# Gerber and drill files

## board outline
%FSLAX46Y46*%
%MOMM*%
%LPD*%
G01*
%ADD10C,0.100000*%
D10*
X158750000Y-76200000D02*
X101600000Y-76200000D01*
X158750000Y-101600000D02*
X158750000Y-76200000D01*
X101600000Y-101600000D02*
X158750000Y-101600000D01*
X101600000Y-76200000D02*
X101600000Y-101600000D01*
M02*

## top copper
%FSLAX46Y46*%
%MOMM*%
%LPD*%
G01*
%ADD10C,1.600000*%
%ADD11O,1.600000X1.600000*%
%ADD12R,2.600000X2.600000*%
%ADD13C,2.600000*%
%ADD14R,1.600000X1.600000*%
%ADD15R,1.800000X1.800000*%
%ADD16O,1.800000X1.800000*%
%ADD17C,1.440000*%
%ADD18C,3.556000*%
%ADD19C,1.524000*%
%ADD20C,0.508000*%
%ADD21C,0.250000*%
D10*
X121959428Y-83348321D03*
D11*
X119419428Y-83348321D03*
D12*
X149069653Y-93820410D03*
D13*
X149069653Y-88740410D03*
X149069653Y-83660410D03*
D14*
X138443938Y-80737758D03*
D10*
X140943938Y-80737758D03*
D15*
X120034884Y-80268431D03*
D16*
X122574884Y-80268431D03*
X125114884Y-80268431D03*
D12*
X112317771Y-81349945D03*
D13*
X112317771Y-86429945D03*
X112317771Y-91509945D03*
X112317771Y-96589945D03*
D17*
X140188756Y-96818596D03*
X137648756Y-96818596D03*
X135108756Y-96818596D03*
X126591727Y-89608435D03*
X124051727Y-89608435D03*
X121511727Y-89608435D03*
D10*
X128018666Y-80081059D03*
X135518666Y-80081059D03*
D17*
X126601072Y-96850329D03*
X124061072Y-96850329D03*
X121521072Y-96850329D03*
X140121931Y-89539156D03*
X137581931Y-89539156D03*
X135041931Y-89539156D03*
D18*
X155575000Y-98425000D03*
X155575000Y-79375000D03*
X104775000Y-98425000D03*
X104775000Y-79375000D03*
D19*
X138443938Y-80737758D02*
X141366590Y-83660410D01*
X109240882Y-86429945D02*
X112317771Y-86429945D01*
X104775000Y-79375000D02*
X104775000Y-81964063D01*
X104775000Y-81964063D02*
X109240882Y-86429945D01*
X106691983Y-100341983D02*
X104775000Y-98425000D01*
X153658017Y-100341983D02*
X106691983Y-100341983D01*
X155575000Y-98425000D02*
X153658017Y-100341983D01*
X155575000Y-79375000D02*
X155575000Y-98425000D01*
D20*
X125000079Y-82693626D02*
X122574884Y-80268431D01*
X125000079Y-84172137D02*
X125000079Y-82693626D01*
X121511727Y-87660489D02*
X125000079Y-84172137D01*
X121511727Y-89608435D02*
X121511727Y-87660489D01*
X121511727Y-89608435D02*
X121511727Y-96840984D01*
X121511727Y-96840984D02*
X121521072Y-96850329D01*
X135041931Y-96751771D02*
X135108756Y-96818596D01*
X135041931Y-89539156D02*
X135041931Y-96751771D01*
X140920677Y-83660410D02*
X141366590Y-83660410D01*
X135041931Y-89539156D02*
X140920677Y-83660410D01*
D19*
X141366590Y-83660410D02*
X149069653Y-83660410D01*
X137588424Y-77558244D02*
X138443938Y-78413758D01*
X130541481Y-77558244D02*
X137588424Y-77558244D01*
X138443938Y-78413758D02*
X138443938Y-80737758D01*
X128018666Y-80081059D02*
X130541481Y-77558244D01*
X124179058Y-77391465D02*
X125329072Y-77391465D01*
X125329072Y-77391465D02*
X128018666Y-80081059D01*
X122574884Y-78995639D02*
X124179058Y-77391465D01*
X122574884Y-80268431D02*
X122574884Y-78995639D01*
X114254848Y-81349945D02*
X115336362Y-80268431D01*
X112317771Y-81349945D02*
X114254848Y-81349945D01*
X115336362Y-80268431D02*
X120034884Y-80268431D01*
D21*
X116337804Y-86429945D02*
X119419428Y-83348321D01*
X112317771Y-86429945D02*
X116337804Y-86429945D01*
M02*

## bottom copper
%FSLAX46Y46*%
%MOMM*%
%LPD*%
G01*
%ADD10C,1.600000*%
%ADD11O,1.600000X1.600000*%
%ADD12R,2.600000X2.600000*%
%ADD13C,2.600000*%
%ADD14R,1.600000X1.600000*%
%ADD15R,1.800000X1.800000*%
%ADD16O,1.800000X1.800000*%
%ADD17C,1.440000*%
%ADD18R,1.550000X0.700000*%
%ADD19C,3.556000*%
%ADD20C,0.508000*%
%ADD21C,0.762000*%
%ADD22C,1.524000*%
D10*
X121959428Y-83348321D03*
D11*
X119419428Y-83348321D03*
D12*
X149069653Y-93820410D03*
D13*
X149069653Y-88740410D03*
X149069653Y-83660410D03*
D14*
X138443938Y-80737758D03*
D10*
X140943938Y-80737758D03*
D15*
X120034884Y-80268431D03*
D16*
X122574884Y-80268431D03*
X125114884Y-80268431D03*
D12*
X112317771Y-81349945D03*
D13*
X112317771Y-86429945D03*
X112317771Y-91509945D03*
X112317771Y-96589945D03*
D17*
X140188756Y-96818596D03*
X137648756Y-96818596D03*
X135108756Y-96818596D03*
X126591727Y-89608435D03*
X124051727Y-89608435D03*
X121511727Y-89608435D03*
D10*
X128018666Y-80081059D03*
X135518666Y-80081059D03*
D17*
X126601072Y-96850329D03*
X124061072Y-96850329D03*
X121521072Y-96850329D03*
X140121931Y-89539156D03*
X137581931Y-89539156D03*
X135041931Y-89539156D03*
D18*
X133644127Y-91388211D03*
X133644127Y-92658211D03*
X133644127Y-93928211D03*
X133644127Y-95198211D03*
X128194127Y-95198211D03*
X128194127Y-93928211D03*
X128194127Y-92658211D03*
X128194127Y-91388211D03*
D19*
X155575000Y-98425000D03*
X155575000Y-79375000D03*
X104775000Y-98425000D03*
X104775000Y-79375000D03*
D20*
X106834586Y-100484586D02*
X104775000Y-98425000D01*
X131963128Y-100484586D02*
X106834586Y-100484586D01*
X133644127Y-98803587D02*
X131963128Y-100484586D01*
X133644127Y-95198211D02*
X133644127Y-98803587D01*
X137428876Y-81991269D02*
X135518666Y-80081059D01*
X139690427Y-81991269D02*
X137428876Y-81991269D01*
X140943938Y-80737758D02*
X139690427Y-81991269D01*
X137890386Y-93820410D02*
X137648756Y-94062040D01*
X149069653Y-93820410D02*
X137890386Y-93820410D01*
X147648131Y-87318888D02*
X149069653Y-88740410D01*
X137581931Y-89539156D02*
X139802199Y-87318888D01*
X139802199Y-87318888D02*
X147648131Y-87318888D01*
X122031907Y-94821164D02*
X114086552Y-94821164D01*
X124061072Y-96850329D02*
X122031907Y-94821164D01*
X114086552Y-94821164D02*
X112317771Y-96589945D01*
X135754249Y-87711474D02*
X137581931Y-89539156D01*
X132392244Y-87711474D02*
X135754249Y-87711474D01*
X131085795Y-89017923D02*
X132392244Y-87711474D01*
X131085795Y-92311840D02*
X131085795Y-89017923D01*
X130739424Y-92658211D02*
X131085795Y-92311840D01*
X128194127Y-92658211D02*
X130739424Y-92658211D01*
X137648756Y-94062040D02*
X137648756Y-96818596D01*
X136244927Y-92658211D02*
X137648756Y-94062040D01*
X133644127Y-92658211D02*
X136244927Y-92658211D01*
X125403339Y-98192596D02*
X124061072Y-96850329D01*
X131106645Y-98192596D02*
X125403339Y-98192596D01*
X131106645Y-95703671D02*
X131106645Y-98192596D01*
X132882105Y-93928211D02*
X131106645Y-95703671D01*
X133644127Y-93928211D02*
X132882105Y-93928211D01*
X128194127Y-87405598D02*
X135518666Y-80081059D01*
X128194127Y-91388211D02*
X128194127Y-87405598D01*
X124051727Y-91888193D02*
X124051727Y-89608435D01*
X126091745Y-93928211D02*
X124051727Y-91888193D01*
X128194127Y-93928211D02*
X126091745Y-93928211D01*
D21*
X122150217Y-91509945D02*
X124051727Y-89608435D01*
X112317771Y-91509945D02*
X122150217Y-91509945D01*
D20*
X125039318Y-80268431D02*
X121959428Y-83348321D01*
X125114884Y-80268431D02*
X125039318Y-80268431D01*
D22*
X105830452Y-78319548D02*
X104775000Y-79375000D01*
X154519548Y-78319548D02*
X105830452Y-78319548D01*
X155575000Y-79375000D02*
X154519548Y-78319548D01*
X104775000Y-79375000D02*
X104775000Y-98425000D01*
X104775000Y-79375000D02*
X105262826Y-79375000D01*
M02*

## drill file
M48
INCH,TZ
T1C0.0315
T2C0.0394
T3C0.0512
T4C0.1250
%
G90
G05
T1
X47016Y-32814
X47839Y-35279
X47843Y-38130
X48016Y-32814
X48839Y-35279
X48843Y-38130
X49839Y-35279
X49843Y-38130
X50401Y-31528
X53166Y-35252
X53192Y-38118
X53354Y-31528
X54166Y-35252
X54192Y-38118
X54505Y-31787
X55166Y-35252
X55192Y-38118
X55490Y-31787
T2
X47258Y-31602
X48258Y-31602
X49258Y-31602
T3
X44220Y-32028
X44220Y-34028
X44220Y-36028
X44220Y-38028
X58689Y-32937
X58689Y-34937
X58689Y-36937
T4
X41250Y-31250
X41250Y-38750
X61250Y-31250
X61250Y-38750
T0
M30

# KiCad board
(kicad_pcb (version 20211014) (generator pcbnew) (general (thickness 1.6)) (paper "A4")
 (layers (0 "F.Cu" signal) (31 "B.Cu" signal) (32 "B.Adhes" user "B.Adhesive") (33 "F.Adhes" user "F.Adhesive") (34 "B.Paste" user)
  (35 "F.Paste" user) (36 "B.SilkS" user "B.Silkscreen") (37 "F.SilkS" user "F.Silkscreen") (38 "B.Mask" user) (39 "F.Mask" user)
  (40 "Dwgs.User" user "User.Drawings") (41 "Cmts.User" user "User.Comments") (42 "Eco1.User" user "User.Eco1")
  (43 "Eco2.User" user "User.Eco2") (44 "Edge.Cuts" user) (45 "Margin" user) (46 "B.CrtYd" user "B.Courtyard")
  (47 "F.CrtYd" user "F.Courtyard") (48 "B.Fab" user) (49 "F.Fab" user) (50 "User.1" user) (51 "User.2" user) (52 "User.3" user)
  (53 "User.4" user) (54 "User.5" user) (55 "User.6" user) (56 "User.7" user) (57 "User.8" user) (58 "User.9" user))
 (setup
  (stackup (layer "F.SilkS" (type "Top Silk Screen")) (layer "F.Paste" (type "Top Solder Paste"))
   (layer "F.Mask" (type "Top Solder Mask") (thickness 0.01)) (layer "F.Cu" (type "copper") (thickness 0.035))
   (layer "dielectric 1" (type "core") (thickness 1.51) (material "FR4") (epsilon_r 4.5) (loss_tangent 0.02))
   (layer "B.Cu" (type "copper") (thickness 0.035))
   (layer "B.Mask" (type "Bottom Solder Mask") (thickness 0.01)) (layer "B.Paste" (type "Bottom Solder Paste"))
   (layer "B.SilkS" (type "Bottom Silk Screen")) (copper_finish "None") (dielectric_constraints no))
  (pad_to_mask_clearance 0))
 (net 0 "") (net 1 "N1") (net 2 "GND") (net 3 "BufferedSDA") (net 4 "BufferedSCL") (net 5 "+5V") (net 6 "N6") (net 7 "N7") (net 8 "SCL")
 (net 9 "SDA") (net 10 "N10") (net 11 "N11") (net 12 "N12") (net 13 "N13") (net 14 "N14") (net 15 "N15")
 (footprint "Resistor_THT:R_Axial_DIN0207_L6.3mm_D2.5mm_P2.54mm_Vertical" (layer "F.Cu") (at 121.959428 83.348321 180)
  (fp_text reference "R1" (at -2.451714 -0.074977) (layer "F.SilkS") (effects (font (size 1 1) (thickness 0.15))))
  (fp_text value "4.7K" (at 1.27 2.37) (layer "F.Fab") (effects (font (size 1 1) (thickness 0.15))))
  (pad "1" thru_hole circle locked (at 0 0 180) (size 1.6 1.6) (drill 0.8) (layers *.Cu *.Mask) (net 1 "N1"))
  (pad "2" thru_hole oval locked (at 2.54 0 180) (size 1.6 1.6) (drill 0.8) (layers *.Cu *.Mask) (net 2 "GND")))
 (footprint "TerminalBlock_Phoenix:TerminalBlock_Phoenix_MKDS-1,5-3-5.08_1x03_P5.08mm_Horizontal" (layer "F.Cu") (at 149.069653 93.82041 90)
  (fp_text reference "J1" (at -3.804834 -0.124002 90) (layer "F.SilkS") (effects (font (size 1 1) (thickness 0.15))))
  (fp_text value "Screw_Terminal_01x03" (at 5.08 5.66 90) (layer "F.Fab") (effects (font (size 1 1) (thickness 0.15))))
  (pad "1" thru_hole rect locked (at 0 0 90) (size 2.6 2.6) (drill 1.3) (layers *.Cu *.Mask) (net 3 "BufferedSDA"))
  (pad "2" thru_hole circle locked (at 5.08 0 90) (size 2.6 2.6) (drill 1.3) (layers *.Cu *.Mask) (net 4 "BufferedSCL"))
  (pad "3" thru_hole circle locked (at 10.16 0 90) (size 2.6 2.6) (drill 1.3) (layers *.Cu *.Mask) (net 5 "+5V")))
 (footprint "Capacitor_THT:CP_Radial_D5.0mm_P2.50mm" (layer "F.Cu") (at 138.443938 80.737758)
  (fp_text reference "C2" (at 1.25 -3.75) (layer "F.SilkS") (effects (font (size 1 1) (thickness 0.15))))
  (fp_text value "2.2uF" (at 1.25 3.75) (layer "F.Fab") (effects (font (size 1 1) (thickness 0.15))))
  (pad "1" thru_hole rect locked (at 0 0) (size 1.6 1.6) (drill 0.8) (layers *.Cu *.Mask) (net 5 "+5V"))
  (pad "2" thru_hole circle locked (at 2.5 0) (size 1.6 1.6) (drill 0.8) (layers *.Cu *.Mask) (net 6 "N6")))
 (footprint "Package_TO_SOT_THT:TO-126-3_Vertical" (layer "F.Cu") (at 120.034884 80.268431)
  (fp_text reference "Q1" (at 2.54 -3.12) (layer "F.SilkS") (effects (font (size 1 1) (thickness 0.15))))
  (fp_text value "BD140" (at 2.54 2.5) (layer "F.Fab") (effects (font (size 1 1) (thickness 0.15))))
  (pad "1" thru_hole rect locked (at 0 0) (size 1.8 1.8) (drill 1) (layers *.Cu *.Mask) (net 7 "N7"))
  (pad "2" thru_hole oval locked (at 2.54 0) (size 1.8 1.8) (drill 1) (layers *.Cu *.Mask) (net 5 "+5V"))
  (pad "3" thru_hole oval locked (at 5.08 0) (size 1.8 1.8) (drill 1) (layers *.Cu *.Mask) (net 1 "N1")))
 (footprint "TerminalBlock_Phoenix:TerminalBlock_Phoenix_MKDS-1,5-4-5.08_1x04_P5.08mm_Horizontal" (layer "F.Cu")
  (at 112.317771 81.349945 -90)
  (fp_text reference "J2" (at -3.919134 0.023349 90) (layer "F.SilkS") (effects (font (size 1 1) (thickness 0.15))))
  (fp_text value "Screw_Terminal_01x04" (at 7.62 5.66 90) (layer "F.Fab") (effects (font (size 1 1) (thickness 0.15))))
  (pad "1" thru_hole rect locked (at 0 0 270) (size 2.6 2.6) (drill 1.3) (layers *.Cu *.Mask) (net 7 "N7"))
  (pad "2" thru_hole circle locked (at 5.08 0 270) (size 2.6 2.6) (drill 1.3) (layers *.Cu *.Mask) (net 2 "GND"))
  (pad "3" thru_hole circle locked (at 10.16 0 270) (size 2.6 2.6) (drill 1.3) (layers *.Cu *.Mask) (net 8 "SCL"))
  (pad "4" thru_hole circle locked (at 15.24 0 270) (size 2.6 2.6) (drill 1.3) (layers *.Cu *.Mask) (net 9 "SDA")))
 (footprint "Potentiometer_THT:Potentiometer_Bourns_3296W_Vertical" (layer "F.Cu") (at 140.188756 96.818596)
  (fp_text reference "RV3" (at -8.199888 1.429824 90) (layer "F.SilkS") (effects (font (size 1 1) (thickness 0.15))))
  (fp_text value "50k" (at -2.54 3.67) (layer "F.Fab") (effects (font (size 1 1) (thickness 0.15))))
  (pad "1" thru_hole circle locked (at 0 0) (size 1.44 1.44) (drill 0.8) (layers *.Cu *.Mask) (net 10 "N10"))
  (pad "2" thru_hole circle locked (at -2.54 0) (size 1.44 1.44) (drill 0.8) (layers *.Cu *.Mask) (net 3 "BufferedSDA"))
  (pad "3" thru_hole circle locked (at -5.08 0) (size 1.44 1.44) (drill 0.8) (layers *.Cu *.Mask) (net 5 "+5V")))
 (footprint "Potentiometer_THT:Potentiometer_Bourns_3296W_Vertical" (layer "F.Cu") (at 126.591727 89.608435)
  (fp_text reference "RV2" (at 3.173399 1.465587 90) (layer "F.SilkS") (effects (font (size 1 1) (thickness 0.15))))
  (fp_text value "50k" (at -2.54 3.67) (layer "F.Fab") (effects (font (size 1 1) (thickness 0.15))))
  (pad "1" thru_hole circle locked (at 0 0) (size 1.44 1.44) (drill 0.8) (layers *.Cu *.Mask) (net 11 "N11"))
  (pad "2" thru_hole circle locked (at -2.54 0) (size 1.44 1.44) (drill 0.8) (layers *.Cu *.Mask) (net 8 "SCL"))
  (pad "3" thru_hole circle locked (at -5.08 0) (size 1.44 1.44) (drill 0.8) (layers *.Cu *.Mask) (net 5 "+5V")))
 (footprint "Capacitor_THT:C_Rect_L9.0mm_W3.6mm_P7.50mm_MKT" (layer "F.Cu") (at 128.018666 80.081059)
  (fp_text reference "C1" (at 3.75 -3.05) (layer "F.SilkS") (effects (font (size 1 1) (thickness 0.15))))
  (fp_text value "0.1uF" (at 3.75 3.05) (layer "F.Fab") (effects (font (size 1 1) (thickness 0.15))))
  (pad "1" thru_hole circle locked (at 0 0) (size 1.6 1.6) (drill 0.8) (layers *.Cu *.Mask) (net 5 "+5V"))
  (pad "2" thru_hole circle locked (at 7.5 0) (size 1.6 1.6) (drill 0.8) (layers *.Cu *.Mask) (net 6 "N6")))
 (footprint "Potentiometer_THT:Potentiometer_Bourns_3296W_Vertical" (layer "F.Cu") (at 126.601072 96.850329)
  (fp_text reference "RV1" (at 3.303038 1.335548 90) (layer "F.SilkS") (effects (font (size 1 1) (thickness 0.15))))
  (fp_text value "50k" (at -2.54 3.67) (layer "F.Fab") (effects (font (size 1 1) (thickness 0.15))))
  (pad "1" thru_hole circle locked (at 0 0) (size 1.44 1.44) (drill 0.8) (layers *.Cu *.Mask) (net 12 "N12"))
  (pad "2" thru_hole circle locked (at -2.54 0) (size 1.44 1.44) (drill 0.8) (layers *.Cu *.Mask) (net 9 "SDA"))
  (pad "3" thru_hole circle locked (at -5.08 0) (size 1.44 1.44) (drill 0.8) (layers *.Cu *.Mask) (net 5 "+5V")))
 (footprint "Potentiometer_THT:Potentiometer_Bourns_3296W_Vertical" (layer "F.Cu") (at 140.121931 89.539156)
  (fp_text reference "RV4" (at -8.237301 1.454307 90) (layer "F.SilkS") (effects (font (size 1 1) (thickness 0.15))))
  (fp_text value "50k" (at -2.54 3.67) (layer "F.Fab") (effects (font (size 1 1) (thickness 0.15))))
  (pad "1" thru_hole circle locked (at 0 0) (size 1.44 1.44) (drill 0.8) (layers *.Cu *.Mask) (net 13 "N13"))
  (pad "2" thru_hole circle locked (at -2.54 0) (size 1.44 1.44) (drill 0.8) (layers *.Cu *.Mask) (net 4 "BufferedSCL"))
  (pad "3" thru_hole circle locked (at -5.08 0) (size 1.44 1.44) (drill 0.8) (layers *.Cu *.Mask) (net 5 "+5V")))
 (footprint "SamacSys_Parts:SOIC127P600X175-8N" (layer "B.Cu") (at 130.919127 93.293211 180)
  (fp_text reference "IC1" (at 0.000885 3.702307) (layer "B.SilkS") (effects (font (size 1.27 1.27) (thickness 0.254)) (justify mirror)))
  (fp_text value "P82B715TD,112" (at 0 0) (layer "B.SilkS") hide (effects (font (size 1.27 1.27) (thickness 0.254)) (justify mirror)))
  (pad "1" smd rect locked (at -2.725 1.905 90) (size 0.7 1.55) (layers "B.Cu" "B.Paste" "B.Mask") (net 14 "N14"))
  (pad "2" smd rect locked (at -2.725 0.635 90) (size 0.7 1.55) (layers "B.Cu" "B.Paste" "B.Mask") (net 3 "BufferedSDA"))
  (pad "3" smd rect locked (at -2.725 -0.635 90) (size 0.7 1.55) (layers "B.Cu" "B.Paste" "B.Mask") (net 9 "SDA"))
  (pad "4" smd rect locked (at -2.725 -1.905 90) (size 0.7 1.55) (layers "B.Cu" "B.Paste" "B.Mask") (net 2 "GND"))
  (pad "5" smd rect locked (at 2.725 -1.905 90) (size 0.7 1.55) (layers "B.Cu" "B.Paste" "B.Mask") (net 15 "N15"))
  (pad "6" smd rect locked (at 2.725 -0.635 90) (size 0.7 1.55) (layers "B.Cu" "B.Paste" "B.Mask") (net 8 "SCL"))
  (pad "7" smd rect locked (at 2.725 0.635 90) (size 0.7 1.55) (layers "B.Cu" "B.Paste" "B.Mask") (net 4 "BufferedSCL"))
  (pad "8" smd rect locked (at 2.725 1.905 90) (size 0.7 1.55) (layers "B.Cu" "B.Paste" "B.Mask") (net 6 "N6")))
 (gr_line (start 101.6 76.2) (end 101.6 101.6) (layer "Edge.Cuts") (width 0.1))
 (gr_line (start 158.75 76.2) (end 101.6 76.2) (layer "Edge.Cuts") (width 0.1))
 (gr_line (start 101.6 101.6) (end 158.75 101.6) (layer "Edge.Cuts") (width 0.1))
 (gr_line (start 158.75 101.6) (end 158.75 76.2) (layer "Edge.Cuts") (width 0.1))
 (segment (start 140.920677 83.66041) (end 141.36659 83.66041) (width 0.508) (layer "F.Cu") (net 5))
 (segment (start 128.018666 80.081059) (end 130.541481 77.558244) (width 1.524) (layer "F.Cu") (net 5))
 (segment (start 122.574884 78.995639) (end 124.179058 77.391465) (width 1.524) (layer "F.Cu") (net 5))
 (segment (start 135.041931 96.751771) (end 135.108756 96.818596) (width 0.508) (layer "F.Cu") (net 5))
 (segment (start 125.000079 84.172137) (end 125.000079 82.693626) (width 0.508) (layer "F.Cu") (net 5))
 (segment (start 125.329072 77.391465) (end 128.018666 80.081059) (width 1.524) (layer "F.Cu") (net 5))
 (segment (start 138.443938 78.413758) (end 138.443938 80.737758) (width 1.524) (layer "F.Cu") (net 5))
 (segment (start 130.541481 77.558244) (end 137.588424 77.558244) (width 1.524) (layer "F.Cu") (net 5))
 (segment (start 124.179058 77.391465) (end 125.329072 77.391465) (width 1.524) (layer "F.Cu") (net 5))
 (segment (start 121.511727 96.840984) (end 121.521072 96.850329) (width 0.508) (layer "F.Cu") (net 5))
 (segment (start 121.511727 87.660489) (end 125.000079 84.172137) (width 0.508) (layer "F.Cu") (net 5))
 (segment (start 125.000079 82.693626) (end 122.574884 80.268431) (width 0.508) (layer "F.Cu") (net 5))
 (segment (start 137.588424 77.558244) (end 138.443938 78.413758) (width 1.524) (layer "F.Cu") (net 5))
 (segment (start 135.041931 89.539156) (end 140.920677 83.66041) (width 0.508) (layer "F.Cu") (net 5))
 (segment (start 141.36659 83.66041) (end 149.069653 83.66041) (width 1.524) (layer "F.Cu") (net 5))
 (segment (start 121.511727 89.608435) (end 121.511727 87.660489) (width 0.508) (layer "F.Cu") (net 5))
 (segment (start 135.041931 89.539156) (end 135.041931 96.751771) (width 0.508) (layer "F.Cu") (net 5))
 (segment (start 121.511727 89.608435) (end 121.511727 96.840984) (width 0.508) (layer "F.Cu") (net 5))
 (segment (start 138.443938 80.737758) (end 141.36659 83.66041) (width 1.524) (layer "F.Cu") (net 5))
 (segment (start 122.574884 80.268431) (end 122.574884 78.995639) (width 1.524) (layer "F.Cu") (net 5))
 (segment (start 140.943938 80.737758) (end 139.690427 81.991269) (width 0.508) (layer "B.Cu") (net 6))
 (segment (start 137.428876 81.991269) (end 135.518666 80.081059) (width 0.508) (layer "B.Cu") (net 6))
 (segment (start 128.194127 91.388211) (end 128.194127 87.405598) (width 0.508) (layer "B.Cu") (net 6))
 (segment (start 139.690427 81.991269) (end 137.428876 81.991269) (width 0.508) (layer "B.Cu") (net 6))
 (segment (start 128.194127 87.405598) (end 135.518666 80.081059) (width 0.508) (layer "B.Cu") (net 6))
 (segment (start 149.069653 93.82041) (end 137.890386 93.82041) (width 0.508) (layer "B.Cu") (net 3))
 (segment (start 137.890386 93.82041) (end 137.648756 94.06204) (width 0.508) (layer "B.Cu") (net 3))
 (segment (start 137.648756 94.06204) (end 137.648756 96.818596) (width 0.508) (layer "B.Cu") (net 3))
 (segment (start 136.244927 92.658211) (end 137.648756 94.06204) (width 0.508) (layer "B.Cu") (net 3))
 (segment (start 133.644127 92.658211) (end 136.244927 92.658211) (width 0.508) (layer "B.Cu") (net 3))
 (segment (start 132.882105 93.928211) (end 131.106645 95.703671) (width 0.508) (layer "B.Cu") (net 9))
 (segment (start 124.061072 96.850329) (end 122.031907 94.821164) (width 0.508) (layer "B.Cu") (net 9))
 (segment (start 122.031907 94.821164) (end 114.086552 94.821164) (width 0.508) (layer "B.Cu") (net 9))
 (segment (start 125.403339 98.192596) (end 124.061072 96.850329) (width 0.508) (layer "B.Cu") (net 9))
 (segment (start 114.086552 94.821164) (end 112.317771 96.589945) (width 0.508) (layer "B.Cu") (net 9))
 (segment (start 133.644127 93.928211) (end 132.882105 93.928211) (width 0.508) (layer "B.Cu") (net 9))
 (segment (start 131.106645 95.703671) (end 131.106645 98.192596) (width 0.508) (layer "B.Cu") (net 9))
 (segment (start 131.106645 98.192596) (end 125.403339 98.192596) (width 0.508) (layer "B.Cu") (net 9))
 (segment (start 104.775 81.964063) (end 109.240882 86.429945) (width 1.524) (layer "F.Cu") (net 2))
 (segment (start 112.317771 86.429945) (end 116.337804 86.429945) (width 0.25) (layer "F.Cu") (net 2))
 (segment (start 153.658017 100.341983) (end 106.691983 100.341983) (width 1.524) (layer "F.Cu") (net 2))
 (segment (start 155.575 79.375) (end 155.575 98.425) (width 1.524) (layer "F.Cu") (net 2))
 (segment (start 104.775 79.375) (end 104.775 81.964063) (width 1.524) (layer "F.Cu") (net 2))
 (segment (start 106.691983 100.341983) (end 104.775 98.425) (width 1.524) (layer "F.Cu") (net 2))
 (segment (start 109.240882 86.429945) (end 112.317771 86.429945) (width 1.524) (layer "F.Cu") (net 2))
 (segment (start 116.337804 86.429945) (end 119.419428 83.348321) (width 0.25) (layer "F.Cu") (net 2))
 (segment (start 155.575 98.425) (end 153.658017 100.341983) (width 1.524) (layer "F.Cu") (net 2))
 (via (at 155.575 98.425) (size 3.556) (drill 3.175) (layers "F.Cu" "B.Cu") (free) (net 2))
 (via (at 104.775 79.375) (size 3.556) (drill 3.175) (layers "F.Cu" "B.Cu") (free) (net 2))
 (via (at 104.775 98.425) (size 3.556) (drill 3.175) (layers "F.Cu" "B.Cu") (free) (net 2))
 (via (at 155.575 79.375) (size 3.556) (drill 3.175) (layers "F.Cu" "B.Cu") (free) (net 2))
 (segment (start 104.775 79.375) (end 105.262826 79.375) (width 1.524) (layer "B.Cu") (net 2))
 (segment (start 133.644127 98.803587) (end 131.963128 100.484586) (width 0.508) (layer "B.Cu") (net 2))
 (segment (start 131.963128 100.484586) (end 106.834586 100.484586) (width 0.508) (layer "B.Cu") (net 2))
 (segment (start 155.575 79.375) (end 154.519548 78.319548) (width 1.524) (layer "B.Cu") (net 2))
 (segment (start 106.834586 100.484586) (end 104.775 98.425) (width 0.508) (layer "B.Cu") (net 2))
 (segment (start 133.644127 95.198211) (end 133.644127 98.803587) (width 0.508) (layer "B.Cu") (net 2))
 (segment (start 104.775 79.375) (end 104.775 98.425) (width 1.524) (layer "B.Cu") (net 2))
 (segment (start 105.830452 78.319548) (end 104.775 79.375) (width 1.524) (layer "B.Cu") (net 2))
 (segment (start 154.519548 78.319548) (end 105.830452 78.319548) (width 1.524) (layer "B.Cu") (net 2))
 (segment (start 112.317771 91.509945) (end 122.150217 91.509945) (width 0.762) (layer "B.Cu") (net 8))
 (segment (start 122.150217 91.509945) (end 124.051727 89.608435) (width 0.762) (layer "B.Cu") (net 8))
 (segment (start 124.051727 91.888193) (end 124.051727 89.608435) (width 0.508) (layer "B.Cu") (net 8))
 (segment (start 126.091745 93.928211) (end 124.051727 91.888193) (width 0.508) (layer "B.Cu") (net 8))
 (segment (start 128.194127 93.928211) (end 126.091745 93.928211) (width 0.508) (layer "B.Cu") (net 8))
 (segment (start 130.739424 92.658211) (end 131.085795 92.31184) (width 0.508) (layer "B.Cu") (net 4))
 (segment (start 128.194127 92.658211) (end 130.739424 92.658211) (width 0.508) (layer "B.Cu") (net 4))
 (segment (start 131.085795 89.017923) (end 132.392244 87.711474) (width 0.508) (layer "B.Cu") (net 4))
 (segment (start 147.648131 87.318888) (end 149.069653 88.74041) (width 0.508) (layer "B.Cu") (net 4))
 (segment (start 135.754249 87.711474) (end 137.581931 89.539156) (width 0.508) (layer "B.Cu") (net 4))
 (segment (start 137.581931 89.539156) (end 139.802199 87.318888) (width 0.508) (layer "B.Cu") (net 4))
 (segment (start 132.392244 87.711474) (end 135.754249 87.711474) (width 0.508) (layer "B.Cu") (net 4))
 (segment (start 139.802199 87.318888) (end 147.648131 87.318888) (width 0.508) (layer "B.Cu") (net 4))
 (segment (start 131.085795 92.31184) (end 131.085795 89.017923) (width 0.508) (layer "B.Cu") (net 4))
 (segment (start 115.336362 80.268431) (end 120.034884 80.268431) (width 1.524) (layer "F.Cu") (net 7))
 (segment (start 112.317771 81.349945) (end 114.254848 81.349945) (width 1.524) (layer "F.Cu") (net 7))
 (segment (start 114.254848 81.349945) (end 115.336362 80.268431) (width 1.524) (layer "F.Cu") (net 7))
 (segment (start 125.039318 80.268431) (end 121.959428 83.348321) (width 0.508) (layer "B.Cu") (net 1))
 (segment (start 125.114884 80.268431) (end 125.039318 80.268431) (width 0.508) (layer "B.Cu") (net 1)))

